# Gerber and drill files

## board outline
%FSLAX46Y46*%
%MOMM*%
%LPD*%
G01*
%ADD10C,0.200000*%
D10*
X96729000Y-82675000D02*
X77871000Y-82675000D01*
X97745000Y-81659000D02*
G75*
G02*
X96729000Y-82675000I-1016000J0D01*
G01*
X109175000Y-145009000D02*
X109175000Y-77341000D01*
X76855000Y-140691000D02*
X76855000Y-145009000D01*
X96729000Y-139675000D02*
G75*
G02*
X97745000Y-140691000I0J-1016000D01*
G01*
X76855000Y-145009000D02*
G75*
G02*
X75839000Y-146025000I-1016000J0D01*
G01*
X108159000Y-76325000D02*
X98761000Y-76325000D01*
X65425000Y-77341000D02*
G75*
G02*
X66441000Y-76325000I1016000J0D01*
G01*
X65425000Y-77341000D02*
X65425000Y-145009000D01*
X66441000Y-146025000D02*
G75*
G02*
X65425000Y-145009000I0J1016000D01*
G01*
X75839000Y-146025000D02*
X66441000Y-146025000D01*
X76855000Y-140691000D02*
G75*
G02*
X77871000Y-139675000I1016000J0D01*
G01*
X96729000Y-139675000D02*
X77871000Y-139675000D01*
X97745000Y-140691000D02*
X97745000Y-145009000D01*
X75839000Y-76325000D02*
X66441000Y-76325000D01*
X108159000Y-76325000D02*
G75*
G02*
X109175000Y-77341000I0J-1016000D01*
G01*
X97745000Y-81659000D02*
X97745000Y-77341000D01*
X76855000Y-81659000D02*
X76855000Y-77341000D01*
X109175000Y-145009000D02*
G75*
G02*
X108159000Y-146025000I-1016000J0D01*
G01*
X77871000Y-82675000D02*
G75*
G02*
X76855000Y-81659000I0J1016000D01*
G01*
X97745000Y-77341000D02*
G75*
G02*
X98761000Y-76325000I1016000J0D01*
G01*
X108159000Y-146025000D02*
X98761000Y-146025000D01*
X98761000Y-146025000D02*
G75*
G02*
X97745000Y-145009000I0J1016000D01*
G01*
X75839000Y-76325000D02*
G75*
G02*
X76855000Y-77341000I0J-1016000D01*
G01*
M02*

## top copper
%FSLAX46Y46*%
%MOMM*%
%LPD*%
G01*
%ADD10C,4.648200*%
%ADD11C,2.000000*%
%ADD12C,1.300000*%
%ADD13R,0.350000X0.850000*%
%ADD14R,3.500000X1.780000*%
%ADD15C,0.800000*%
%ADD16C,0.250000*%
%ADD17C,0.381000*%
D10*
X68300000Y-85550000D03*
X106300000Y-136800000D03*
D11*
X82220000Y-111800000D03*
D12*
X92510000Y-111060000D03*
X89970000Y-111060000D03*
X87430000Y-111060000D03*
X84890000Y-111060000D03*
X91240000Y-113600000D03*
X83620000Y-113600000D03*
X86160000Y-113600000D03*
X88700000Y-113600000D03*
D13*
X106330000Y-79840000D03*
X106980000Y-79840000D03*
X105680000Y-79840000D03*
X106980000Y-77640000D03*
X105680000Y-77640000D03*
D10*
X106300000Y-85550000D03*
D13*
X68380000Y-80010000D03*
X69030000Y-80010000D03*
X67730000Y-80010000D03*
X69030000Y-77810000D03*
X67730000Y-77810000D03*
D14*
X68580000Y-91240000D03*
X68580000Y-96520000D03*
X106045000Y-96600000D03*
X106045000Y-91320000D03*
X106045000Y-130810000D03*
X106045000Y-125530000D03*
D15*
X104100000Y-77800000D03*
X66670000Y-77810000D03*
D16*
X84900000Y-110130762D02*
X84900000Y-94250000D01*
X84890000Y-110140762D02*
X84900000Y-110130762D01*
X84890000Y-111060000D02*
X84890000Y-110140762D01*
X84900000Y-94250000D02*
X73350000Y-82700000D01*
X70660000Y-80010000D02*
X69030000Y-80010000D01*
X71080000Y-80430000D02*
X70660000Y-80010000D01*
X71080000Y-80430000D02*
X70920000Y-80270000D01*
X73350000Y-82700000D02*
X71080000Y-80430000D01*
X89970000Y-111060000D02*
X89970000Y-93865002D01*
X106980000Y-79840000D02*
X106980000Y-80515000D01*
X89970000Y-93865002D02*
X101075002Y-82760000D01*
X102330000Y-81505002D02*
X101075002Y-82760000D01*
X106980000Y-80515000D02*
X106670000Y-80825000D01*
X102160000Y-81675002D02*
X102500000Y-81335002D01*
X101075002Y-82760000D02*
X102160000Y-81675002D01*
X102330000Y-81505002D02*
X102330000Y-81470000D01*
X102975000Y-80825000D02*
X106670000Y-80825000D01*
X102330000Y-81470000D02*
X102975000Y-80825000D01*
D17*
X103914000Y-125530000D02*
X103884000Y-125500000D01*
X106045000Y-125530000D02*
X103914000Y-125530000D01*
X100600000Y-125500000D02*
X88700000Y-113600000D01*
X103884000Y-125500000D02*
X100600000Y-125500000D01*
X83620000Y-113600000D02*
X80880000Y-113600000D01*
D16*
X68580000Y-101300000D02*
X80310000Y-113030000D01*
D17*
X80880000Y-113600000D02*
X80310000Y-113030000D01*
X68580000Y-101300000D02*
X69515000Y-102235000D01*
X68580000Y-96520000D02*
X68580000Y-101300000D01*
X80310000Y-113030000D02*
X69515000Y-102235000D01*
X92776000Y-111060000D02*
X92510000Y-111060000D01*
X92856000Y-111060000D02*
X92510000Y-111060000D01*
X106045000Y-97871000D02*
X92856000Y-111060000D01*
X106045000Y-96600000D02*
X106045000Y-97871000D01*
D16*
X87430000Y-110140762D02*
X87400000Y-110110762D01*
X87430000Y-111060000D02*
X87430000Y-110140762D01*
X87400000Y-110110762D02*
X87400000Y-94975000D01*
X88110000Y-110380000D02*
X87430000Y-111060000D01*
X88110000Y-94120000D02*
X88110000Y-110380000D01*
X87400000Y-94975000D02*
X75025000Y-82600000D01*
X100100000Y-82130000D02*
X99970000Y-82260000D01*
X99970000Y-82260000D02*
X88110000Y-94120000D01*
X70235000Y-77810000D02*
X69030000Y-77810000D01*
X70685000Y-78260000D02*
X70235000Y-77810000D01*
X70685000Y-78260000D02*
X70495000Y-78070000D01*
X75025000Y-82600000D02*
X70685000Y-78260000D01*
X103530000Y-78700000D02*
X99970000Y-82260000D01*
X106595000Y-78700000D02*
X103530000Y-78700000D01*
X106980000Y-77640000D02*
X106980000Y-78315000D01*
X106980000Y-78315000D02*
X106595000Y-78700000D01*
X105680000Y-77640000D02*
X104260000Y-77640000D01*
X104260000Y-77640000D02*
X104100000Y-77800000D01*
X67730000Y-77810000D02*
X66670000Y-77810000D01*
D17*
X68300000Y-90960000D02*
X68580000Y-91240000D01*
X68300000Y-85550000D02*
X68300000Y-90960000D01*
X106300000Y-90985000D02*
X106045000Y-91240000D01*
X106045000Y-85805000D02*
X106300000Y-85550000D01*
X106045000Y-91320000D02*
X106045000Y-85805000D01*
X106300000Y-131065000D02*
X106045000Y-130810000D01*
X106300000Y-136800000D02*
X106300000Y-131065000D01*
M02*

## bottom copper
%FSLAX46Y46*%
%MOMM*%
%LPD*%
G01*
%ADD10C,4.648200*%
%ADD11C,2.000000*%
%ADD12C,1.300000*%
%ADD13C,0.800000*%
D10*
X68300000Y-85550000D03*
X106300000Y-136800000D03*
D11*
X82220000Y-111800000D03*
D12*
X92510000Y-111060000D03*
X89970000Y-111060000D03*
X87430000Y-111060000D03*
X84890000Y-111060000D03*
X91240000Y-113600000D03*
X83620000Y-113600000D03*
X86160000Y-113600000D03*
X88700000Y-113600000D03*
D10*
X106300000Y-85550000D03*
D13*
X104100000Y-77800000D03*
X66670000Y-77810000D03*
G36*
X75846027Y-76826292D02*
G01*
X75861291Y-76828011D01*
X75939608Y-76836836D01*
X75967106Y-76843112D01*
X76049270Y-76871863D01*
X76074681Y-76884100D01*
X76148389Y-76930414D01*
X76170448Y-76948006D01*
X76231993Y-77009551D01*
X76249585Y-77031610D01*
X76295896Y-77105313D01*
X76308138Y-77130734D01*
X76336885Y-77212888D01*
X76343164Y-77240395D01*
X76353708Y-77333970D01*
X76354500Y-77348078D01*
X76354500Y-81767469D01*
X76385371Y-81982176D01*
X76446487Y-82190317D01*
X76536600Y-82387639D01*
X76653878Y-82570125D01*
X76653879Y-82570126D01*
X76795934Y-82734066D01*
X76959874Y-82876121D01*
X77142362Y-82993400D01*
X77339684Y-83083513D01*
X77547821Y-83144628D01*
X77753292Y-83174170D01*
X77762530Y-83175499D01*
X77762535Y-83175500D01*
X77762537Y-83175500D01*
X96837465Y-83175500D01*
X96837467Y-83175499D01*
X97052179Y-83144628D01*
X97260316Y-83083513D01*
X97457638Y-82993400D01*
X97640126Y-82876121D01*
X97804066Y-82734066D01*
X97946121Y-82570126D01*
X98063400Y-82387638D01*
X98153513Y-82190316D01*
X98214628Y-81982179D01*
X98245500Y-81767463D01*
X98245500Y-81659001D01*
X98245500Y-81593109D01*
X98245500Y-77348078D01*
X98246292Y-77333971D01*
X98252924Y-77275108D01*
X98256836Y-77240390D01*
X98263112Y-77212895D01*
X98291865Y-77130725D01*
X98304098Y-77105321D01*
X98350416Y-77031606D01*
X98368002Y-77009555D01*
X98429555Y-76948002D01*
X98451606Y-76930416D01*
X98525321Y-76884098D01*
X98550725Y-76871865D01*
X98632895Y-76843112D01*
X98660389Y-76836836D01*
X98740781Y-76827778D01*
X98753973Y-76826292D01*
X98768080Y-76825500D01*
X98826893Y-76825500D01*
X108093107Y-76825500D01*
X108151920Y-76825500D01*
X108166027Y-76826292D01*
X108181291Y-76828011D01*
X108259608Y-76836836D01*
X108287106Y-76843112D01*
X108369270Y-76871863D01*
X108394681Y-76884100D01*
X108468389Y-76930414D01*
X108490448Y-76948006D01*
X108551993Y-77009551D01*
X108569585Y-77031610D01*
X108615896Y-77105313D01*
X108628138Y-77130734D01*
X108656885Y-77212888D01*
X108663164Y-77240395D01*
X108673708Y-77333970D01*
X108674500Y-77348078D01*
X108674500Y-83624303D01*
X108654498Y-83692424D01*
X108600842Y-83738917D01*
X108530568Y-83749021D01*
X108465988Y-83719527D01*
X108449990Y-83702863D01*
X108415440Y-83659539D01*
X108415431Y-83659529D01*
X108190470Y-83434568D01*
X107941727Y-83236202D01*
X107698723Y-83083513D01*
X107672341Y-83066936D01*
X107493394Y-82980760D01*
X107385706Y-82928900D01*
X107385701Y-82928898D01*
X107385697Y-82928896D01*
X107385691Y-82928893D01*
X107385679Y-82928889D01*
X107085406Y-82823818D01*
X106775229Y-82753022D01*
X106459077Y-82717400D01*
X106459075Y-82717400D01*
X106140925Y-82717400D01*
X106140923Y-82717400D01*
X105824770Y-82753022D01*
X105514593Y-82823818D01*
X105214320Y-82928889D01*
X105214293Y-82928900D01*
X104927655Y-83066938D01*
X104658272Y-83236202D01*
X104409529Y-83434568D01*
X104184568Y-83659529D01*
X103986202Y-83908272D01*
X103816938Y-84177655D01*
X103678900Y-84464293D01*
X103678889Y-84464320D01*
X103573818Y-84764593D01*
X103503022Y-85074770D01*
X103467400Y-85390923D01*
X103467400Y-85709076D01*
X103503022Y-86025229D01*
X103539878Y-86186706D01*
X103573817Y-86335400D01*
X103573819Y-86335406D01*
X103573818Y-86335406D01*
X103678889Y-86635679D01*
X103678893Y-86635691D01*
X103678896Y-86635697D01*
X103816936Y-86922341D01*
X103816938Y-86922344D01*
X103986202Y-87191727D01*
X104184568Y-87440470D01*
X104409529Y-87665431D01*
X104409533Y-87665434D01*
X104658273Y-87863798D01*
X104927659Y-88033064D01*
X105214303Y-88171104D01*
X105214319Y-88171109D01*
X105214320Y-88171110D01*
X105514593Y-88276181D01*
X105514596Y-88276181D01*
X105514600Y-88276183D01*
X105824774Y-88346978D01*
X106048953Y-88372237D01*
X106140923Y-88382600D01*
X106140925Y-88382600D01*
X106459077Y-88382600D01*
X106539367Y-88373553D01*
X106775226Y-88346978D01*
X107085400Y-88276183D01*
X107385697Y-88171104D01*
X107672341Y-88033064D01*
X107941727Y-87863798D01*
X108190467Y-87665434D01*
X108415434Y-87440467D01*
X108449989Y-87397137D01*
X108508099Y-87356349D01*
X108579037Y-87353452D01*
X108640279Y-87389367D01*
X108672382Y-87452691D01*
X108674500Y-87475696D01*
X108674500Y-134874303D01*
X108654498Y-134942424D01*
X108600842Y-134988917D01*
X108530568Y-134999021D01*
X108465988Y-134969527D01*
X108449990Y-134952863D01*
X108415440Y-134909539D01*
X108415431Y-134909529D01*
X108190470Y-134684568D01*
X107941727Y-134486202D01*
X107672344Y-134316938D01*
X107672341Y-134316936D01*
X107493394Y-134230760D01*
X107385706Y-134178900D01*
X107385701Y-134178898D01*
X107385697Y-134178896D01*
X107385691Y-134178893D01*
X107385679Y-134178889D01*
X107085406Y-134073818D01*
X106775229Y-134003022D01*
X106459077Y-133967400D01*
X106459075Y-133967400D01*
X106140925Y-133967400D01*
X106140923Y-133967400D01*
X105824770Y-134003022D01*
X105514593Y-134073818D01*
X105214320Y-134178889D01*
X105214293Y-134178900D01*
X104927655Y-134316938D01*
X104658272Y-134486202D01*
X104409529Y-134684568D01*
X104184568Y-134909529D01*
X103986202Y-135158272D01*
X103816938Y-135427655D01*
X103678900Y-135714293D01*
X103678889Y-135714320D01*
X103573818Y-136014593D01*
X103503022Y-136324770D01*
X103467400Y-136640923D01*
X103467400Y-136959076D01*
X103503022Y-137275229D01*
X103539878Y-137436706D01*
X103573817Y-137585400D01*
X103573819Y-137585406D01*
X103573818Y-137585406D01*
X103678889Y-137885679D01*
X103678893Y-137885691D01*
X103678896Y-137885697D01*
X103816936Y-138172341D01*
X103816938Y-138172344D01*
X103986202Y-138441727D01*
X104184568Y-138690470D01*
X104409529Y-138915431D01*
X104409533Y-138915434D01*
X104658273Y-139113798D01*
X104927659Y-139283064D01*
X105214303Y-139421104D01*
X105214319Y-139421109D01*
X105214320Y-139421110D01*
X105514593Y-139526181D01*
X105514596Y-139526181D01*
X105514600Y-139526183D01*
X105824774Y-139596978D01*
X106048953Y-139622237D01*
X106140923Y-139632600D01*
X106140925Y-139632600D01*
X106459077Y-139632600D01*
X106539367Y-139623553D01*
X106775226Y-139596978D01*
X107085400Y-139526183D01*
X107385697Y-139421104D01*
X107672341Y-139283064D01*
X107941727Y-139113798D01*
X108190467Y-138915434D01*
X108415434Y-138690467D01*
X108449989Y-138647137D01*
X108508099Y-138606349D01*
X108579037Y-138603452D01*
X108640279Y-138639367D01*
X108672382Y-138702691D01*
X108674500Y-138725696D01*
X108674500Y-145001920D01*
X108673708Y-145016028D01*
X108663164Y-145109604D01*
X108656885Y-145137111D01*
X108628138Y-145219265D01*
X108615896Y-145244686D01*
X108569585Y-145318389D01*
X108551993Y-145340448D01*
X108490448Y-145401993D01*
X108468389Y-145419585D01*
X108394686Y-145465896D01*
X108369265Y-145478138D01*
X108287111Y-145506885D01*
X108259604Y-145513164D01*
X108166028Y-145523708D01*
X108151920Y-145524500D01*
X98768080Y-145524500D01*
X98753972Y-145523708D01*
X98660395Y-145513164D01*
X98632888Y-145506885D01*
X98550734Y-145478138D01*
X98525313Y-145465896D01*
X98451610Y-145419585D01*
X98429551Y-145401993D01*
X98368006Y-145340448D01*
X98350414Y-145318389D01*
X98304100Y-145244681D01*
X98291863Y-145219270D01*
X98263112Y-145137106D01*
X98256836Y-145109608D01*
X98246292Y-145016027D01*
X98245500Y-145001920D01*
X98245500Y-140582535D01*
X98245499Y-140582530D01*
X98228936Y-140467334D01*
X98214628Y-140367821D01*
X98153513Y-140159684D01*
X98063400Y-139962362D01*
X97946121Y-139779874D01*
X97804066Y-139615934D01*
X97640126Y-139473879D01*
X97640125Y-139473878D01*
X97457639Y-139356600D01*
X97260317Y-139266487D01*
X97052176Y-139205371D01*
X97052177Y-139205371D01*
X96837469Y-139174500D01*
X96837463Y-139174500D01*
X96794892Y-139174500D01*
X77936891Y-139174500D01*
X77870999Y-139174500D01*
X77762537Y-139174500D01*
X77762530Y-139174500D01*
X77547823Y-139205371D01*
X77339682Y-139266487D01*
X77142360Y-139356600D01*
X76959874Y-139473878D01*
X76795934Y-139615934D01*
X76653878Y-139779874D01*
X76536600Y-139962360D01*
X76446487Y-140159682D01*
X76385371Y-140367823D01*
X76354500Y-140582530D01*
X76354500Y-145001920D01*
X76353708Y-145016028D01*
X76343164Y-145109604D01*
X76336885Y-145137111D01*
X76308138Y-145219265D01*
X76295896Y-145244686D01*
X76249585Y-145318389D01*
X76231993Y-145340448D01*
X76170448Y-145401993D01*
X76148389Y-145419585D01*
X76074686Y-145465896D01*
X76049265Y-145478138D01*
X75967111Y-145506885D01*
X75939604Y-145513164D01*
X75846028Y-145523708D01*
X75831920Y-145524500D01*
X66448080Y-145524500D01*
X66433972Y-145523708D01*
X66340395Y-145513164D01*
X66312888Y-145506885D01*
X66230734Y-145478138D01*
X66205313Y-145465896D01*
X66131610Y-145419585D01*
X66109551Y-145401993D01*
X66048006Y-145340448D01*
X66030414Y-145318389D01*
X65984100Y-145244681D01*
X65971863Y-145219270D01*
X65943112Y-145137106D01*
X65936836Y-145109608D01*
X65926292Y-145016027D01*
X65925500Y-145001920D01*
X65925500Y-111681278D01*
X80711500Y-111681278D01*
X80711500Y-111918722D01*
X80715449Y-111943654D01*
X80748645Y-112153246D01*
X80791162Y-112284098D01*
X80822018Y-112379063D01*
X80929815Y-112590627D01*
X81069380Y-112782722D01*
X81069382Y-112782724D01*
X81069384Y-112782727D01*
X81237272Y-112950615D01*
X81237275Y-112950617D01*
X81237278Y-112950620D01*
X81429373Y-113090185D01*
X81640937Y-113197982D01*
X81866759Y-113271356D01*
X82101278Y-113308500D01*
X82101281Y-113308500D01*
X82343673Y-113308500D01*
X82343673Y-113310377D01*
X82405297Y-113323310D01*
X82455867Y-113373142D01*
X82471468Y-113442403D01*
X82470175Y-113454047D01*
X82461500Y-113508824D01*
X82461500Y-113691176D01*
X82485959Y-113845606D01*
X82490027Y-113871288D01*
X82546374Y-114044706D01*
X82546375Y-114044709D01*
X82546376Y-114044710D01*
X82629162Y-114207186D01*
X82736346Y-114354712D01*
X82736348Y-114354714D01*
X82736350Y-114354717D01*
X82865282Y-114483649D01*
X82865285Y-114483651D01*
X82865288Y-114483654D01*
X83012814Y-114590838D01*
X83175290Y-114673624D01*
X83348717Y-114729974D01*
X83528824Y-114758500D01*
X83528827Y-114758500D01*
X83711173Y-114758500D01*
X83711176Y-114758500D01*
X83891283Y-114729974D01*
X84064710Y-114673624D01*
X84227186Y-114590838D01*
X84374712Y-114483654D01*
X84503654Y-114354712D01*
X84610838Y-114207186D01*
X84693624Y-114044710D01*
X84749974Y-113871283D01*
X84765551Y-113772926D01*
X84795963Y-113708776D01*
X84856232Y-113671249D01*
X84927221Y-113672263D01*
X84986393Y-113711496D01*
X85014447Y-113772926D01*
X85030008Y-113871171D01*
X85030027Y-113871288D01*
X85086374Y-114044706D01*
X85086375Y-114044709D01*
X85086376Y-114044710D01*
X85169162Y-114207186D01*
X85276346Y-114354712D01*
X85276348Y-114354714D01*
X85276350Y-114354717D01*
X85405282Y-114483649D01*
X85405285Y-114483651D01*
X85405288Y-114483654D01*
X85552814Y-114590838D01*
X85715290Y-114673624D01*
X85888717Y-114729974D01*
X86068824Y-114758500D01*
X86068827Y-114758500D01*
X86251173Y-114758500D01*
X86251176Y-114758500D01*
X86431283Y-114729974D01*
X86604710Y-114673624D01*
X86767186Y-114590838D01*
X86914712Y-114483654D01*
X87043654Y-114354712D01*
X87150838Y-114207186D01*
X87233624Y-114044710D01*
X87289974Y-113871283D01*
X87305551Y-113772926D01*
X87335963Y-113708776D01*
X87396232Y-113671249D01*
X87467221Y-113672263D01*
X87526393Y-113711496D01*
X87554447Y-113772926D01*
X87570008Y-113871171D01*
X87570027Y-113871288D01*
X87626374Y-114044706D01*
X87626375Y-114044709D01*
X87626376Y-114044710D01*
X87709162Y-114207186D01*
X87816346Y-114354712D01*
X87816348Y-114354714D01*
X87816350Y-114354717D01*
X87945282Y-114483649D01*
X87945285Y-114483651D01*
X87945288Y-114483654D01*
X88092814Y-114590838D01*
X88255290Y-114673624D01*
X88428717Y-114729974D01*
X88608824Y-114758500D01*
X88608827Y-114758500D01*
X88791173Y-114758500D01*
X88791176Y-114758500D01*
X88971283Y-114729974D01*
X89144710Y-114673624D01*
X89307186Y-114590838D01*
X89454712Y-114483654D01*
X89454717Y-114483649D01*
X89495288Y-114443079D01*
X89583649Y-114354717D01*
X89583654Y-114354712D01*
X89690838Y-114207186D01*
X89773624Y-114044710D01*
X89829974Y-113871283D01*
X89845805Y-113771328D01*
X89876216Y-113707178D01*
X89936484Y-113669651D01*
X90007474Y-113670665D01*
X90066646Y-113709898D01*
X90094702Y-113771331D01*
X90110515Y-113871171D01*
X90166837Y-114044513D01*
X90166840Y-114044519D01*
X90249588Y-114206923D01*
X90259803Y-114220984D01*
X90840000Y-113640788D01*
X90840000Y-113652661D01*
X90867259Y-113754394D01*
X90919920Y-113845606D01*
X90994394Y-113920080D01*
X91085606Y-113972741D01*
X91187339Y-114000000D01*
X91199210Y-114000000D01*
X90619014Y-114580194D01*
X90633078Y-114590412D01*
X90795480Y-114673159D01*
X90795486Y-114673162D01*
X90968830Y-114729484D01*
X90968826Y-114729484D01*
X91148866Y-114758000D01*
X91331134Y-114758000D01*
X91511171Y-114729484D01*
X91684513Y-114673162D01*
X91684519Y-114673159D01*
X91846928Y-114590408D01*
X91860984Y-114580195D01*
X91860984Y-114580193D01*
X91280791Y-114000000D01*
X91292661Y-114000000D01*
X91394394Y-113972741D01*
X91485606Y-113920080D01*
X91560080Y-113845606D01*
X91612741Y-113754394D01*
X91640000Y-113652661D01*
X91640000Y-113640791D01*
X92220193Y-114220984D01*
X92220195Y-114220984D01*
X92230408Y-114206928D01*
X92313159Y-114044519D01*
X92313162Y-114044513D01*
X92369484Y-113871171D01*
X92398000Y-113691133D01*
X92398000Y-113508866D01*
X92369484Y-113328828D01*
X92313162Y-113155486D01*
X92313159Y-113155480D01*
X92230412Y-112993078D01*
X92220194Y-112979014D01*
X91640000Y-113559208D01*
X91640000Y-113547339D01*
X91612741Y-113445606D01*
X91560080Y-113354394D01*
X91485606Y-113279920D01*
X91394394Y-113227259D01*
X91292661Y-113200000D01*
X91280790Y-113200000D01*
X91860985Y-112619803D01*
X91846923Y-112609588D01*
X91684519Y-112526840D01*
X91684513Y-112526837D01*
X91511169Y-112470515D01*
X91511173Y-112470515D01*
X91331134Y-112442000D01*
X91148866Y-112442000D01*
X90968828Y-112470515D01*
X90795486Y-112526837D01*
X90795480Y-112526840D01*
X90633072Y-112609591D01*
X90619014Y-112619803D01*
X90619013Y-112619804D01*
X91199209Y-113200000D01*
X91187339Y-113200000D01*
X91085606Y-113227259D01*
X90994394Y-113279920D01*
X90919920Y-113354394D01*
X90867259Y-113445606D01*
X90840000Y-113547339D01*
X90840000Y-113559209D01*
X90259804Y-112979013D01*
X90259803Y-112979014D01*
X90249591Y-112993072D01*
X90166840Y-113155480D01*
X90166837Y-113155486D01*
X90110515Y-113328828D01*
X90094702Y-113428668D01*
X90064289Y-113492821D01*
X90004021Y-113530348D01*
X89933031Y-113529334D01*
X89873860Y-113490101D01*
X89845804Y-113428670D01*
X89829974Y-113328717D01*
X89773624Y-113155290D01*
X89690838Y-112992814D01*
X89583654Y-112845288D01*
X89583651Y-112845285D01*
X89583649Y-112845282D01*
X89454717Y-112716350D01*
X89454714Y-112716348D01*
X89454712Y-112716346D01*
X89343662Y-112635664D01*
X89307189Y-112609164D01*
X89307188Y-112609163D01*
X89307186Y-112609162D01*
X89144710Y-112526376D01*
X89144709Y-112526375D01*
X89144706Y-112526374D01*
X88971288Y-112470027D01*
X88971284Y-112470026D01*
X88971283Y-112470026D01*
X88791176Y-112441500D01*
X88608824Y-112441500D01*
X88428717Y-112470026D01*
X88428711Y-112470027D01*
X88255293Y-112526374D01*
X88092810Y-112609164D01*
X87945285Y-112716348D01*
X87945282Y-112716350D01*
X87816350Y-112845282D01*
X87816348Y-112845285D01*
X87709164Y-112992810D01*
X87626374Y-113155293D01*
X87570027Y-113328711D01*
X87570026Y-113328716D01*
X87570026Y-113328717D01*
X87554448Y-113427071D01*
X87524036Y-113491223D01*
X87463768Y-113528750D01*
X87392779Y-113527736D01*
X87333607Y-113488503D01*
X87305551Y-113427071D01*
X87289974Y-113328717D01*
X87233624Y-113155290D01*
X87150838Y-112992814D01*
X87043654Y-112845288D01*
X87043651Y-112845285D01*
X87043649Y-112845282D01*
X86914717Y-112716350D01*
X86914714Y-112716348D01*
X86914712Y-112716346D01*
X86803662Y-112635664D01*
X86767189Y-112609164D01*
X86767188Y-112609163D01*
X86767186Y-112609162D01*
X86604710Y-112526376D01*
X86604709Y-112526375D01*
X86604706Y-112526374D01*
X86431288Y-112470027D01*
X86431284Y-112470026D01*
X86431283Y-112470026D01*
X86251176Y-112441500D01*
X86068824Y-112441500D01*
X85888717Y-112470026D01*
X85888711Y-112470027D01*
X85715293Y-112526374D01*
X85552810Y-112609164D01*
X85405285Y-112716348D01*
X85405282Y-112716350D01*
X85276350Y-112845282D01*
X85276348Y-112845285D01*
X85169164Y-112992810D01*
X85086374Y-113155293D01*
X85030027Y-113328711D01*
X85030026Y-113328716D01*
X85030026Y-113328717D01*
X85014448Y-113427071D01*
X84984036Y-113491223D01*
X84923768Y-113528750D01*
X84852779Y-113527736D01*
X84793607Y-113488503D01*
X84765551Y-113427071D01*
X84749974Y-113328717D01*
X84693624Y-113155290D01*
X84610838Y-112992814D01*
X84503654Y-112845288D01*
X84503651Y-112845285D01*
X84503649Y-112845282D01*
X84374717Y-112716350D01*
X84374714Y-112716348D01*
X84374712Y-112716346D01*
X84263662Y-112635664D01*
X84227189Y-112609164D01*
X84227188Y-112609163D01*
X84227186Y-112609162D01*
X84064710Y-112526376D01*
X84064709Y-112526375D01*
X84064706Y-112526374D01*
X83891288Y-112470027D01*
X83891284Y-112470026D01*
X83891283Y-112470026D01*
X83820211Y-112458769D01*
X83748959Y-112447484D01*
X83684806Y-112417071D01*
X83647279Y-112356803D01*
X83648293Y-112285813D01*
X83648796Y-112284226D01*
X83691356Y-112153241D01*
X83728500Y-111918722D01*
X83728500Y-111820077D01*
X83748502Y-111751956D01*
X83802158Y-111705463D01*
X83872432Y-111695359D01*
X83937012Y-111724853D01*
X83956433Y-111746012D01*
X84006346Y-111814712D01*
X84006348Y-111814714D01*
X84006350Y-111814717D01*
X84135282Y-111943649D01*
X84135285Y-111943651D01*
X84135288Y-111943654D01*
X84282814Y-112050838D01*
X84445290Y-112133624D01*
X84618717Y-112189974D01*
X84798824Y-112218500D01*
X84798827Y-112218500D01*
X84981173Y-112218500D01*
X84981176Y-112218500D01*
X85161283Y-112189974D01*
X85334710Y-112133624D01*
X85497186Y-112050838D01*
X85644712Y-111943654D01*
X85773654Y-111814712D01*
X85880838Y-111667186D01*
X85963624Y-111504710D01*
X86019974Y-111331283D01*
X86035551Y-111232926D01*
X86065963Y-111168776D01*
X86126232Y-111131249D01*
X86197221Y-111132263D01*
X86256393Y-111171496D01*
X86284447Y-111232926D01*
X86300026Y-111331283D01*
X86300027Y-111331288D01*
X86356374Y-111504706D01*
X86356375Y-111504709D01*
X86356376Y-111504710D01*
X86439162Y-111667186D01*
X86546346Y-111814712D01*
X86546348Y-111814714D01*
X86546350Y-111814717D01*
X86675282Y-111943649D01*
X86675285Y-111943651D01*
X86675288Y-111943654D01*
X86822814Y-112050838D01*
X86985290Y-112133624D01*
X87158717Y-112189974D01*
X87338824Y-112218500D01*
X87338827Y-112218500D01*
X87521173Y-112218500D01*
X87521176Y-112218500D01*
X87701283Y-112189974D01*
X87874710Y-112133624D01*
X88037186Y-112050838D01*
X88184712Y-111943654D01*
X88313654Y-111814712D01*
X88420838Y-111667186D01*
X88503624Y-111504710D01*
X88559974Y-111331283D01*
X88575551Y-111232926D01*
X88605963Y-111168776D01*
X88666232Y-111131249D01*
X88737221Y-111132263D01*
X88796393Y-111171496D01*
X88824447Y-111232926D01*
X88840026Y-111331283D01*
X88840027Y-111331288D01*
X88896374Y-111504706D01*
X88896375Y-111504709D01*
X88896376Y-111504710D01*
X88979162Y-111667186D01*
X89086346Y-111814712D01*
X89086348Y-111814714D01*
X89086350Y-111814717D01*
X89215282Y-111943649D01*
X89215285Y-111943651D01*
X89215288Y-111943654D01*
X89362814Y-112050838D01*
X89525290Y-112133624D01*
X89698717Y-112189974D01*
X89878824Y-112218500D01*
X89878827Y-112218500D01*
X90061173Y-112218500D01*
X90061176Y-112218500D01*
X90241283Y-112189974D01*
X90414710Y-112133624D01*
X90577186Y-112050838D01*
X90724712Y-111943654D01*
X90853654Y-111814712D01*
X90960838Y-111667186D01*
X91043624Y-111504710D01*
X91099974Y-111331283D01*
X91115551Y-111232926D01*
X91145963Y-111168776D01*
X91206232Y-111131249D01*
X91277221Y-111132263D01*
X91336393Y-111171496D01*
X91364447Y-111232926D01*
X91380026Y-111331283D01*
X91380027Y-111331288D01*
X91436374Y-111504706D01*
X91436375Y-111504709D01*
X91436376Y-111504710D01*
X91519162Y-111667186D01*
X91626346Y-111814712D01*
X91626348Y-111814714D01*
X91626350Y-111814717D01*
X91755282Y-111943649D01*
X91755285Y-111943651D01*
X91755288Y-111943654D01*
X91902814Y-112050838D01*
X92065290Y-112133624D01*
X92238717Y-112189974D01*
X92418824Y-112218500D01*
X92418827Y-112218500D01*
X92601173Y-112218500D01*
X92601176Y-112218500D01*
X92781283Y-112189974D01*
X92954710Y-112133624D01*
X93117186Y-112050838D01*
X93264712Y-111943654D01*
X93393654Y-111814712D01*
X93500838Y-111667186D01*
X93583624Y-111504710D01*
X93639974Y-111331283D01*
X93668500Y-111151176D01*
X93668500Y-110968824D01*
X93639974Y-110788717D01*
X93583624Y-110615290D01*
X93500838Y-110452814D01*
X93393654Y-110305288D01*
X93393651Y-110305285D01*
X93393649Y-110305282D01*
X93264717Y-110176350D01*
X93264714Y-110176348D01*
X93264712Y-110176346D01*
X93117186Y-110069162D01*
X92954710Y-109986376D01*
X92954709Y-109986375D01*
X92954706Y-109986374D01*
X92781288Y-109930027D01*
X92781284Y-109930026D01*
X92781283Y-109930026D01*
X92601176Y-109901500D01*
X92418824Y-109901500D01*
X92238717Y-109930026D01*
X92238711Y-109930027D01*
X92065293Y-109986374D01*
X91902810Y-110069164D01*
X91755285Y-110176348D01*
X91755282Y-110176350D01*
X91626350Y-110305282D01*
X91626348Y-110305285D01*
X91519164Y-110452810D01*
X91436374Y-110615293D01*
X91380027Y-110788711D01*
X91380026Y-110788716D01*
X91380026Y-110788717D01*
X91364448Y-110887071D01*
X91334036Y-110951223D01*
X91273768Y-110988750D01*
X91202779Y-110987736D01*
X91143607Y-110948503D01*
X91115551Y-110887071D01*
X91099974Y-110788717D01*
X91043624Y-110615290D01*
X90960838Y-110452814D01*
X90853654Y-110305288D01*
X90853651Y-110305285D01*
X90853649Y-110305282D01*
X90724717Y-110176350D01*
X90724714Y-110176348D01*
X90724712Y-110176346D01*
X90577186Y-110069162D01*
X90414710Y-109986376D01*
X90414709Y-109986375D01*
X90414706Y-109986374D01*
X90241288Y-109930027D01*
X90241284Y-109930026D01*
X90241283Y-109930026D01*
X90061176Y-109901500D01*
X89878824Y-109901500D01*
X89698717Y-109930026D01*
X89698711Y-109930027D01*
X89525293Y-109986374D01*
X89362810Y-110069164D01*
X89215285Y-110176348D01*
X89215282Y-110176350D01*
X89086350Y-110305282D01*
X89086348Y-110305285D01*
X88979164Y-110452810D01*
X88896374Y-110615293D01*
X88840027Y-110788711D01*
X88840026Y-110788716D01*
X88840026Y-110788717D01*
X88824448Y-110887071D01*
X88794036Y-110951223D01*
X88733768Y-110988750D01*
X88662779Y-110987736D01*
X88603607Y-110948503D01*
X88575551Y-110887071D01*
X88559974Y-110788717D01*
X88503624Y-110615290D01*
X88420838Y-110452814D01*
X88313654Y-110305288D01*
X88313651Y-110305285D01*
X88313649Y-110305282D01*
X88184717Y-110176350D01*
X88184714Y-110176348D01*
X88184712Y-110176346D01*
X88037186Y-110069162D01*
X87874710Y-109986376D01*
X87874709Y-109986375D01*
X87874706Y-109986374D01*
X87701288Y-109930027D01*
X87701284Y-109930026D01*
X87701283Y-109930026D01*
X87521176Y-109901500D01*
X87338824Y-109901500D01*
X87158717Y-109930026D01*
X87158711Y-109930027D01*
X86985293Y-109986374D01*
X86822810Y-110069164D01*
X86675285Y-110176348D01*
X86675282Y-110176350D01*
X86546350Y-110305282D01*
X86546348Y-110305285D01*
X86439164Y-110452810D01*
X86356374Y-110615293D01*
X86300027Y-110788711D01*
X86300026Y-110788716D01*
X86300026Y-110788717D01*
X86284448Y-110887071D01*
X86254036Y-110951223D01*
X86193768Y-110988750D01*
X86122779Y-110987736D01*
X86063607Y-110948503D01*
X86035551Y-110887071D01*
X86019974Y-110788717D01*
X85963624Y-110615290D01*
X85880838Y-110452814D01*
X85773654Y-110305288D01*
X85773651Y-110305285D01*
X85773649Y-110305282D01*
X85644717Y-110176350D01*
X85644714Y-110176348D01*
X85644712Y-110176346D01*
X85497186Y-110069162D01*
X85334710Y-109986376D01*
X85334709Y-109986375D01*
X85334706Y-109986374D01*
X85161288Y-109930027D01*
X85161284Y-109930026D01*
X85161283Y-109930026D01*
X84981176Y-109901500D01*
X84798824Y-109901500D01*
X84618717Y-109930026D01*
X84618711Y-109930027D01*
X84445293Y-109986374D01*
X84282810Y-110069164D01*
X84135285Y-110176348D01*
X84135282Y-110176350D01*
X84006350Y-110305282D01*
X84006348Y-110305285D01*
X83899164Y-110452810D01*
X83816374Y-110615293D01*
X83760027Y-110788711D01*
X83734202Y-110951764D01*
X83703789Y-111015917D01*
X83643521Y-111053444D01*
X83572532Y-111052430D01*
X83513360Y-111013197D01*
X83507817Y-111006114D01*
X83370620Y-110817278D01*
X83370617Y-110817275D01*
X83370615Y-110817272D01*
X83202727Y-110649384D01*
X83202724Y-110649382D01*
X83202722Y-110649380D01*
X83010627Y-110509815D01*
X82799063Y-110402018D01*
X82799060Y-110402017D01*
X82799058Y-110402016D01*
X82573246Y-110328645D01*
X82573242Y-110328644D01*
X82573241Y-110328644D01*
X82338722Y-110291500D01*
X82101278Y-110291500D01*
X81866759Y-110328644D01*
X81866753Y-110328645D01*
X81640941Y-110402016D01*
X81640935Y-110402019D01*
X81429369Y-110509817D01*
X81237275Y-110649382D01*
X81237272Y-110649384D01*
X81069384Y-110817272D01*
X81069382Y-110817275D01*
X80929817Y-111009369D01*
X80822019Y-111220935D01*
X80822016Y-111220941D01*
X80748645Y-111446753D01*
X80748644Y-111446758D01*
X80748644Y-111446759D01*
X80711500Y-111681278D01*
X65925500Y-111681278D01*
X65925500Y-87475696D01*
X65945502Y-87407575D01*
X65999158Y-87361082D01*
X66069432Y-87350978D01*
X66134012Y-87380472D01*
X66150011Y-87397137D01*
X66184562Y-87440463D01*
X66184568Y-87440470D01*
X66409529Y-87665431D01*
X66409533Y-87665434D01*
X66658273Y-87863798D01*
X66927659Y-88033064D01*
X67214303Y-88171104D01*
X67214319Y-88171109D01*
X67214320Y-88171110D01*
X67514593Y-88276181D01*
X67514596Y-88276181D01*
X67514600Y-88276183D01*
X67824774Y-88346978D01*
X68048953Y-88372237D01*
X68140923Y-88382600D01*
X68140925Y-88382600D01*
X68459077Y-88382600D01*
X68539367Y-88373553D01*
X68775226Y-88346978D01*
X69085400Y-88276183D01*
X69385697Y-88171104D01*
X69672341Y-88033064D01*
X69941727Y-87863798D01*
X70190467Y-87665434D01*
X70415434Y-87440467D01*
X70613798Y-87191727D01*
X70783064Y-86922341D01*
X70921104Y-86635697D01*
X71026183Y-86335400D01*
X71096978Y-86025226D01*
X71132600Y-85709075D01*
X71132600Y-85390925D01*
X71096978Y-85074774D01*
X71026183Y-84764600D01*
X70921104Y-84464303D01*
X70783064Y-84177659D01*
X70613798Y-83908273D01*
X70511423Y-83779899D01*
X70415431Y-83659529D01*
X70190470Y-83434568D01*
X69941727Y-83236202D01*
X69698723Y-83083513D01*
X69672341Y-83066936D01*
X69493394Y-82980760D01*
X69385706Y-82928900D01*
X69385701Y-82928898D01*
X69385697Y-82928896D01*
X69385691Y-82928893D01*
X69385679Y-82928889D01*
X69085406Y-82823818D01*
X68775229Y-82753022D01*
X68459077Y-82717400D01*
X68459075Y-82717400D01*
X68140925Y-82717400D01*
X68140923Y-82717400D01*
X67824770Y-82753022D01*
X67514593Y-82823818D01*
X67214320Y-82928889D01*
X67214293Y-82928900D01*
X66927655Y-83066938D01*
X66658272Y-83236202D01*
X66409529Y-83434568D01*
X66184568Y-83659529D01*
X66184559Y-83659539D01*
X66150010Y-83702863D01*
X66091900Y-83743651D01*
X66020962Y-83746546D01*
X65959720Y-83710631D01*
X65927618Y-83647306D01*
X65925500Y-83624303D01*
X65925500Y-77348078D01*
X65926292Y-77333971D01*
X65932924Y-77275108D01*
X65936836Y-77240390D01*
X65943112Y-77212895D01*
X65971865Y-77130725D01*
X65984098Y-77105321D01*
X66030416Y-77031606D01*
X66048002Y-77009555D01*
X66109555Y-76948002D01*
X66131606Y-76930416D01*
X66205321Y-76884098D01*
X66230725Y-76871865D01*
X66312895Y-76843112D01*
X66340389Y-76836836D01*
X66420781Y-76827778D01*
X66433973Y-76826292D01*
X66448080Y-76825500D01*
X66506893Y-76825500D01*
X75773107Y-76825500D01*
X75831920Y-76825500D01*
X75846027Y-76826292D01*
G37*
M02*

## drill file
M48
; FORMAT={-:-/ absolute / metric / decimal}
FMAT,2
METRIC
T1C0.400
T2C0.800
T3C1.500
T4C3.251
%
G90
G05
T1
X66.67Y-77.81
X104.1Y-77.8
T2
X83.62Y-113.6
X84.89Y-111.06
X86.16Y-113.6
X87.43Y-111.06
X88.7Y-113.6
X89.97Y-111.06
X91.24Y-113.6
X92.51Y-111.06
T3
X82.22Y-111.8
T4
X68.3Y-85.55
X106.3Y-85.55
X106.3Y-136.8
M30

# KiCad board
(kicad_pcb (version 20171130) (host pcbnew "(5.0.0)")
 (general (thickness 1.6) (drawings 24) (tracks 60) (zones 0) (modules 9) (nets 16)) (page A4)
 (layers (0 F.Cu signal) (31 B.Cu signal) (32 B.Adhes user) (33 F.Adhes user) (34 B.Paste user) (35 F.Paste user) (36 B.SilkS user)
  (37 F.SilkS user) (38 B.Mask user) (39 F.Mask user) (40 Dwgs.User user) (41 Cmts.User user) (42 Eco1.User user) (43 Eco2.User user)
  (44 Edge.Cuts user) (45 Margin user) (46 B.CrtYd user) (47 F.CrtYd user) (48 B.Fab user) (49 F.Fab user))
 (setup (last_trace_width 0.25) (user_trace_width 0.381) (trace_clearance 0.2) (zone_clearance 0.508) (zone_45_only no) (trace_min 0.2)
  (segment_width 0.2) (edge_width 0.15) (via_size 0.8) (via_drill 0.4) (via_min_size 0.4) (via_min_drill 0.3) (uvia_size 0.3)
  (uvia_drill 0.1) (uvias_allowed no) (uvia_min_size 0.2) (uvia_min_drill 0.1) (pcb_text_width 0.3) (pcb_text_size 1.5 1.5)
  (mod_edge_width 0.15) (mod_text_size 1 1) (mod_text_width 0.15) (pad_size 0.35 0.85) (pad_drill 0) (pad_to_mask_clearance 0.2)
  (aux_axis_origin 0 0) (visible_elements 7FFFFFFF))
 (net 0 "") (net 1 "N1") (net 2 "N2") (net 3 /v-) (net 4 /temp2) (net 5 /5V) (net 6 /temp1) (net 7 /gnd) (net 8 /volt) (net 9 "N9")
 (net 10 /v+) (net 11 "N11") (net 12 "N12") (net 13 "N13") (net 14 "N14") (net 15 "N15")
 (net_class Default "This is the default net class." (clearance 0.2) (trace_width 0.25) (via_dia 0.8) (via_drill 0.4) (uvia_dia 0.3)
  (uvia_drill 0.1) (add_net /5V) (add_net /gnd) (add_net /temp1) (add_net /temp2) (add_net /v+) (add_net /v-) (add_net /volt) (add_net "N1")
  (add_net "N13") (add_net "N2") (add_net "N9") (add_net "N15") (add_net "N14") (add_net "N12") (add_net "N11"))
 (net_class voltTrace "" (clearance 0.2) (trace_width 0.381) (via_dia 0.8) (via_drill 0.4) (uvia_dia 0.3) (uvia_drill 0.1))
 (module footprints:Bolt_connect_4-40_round (layer F.Cu) (at 68.3 85.55)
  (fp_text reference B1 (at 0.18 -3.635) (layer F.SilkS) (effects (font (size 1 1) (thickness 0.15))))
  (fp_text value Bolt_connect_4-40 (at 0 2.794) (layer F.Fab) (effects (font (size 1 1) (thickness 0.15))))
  (pad 1 thru_hole circle (at 0 0) (size 4.6482 4.6482) (drill 3.2512) (layers *.Cu *.Mask) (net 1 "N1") (clearance 0.508)))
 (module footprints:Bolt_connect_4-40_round (layer F.Cu) (at 106.3 136.8)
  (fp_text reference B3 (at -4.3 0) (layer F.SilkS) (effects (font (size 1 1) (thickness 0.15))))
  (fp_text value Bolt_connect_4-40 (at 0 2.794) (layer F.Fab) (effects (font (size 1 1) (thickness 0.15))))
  (pad 1 thru_hole circle (at 0 0) (size 4.6482 4.6482) (drill 3.2512) (layers *.Cu *.Mask) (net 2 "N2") (clearance 0.508)))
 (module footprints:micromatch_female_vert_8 (layer F.Cu) (at 88.7 113.6 90)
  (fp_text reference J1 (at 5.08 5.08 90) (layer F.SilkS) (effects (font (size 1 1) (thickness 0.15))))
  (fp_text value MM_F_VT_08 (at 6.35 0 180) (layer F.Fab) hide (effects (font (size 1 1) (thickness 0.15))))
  (pad 9 thru_hole circle (at 1.8 -6.48 90) (size 2 2) (drill 1.5) (layers *.Cu *.Mask))
  (pad 8 thru_hole circle (at 2.54 3.81 90) (size 1.3 1.3) (drill 0.8) (layers *.Cu *.Mask) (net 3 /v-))
  (pad 6 thru_hole circle (at 2.54 1.27 90) (size 1.3 1.3) (drill 0.8) (layers *.Cu *.Mask) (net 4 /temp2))
  (pad 4 thru_hole circle (at 2.54 -1.27 90) (size 1.3 1.3) (drill 0.8) (layers *.Cu *.Mask) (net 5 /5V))
  (pad 2 thru_hole circle (at 2.54 -3.81 90) (size 1.3 1.3) (drill 0.8) (layers *.Cu *.Mask) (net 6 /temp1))
  (pad 7 thru_hole circle (at 0 2.54 90) (size 1.3 1.3) (drill 0.8) (layers *.Cu *.Mask) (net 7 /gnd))
  (pad 1 thru_hole circle (at 0 -5.08 90) (size 1.3 1.3) (drill 0.8) (layers *.Cu *.Mask) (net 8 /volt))
  (pad 3 thru_hole circle (at 0 -2.54 90) (size 1.3 1.3) (drill 0.8) (layers *.Cu *.Mask) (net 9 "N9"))
  (pad 5 thru_hole circle (at 0 0 90) (size 1.3 1.3) (drill 0.8) (layers *.Cu *.Mask) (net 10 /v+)))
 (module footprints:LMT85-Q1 (layer F.Cu) (at 105.68 79.84)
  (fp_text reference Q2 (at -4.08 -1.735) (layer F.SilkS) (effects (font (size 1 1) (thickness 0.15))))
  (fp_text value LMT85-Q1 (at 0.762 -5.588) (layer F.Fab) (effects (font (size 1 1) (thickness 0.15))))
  (pad 3 smd rect (at 0.65 0) (size 0.35 0.85) (layers F.Cu F.Paste F.Mask) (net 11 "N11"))
  (pad 4 smd rect (at 1.3 0) (size 0.35 0.85) (layers F.Cu F.Paste F.Mask) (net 4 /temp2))
  (pad 2 smd rect (at 0 0) (size 0.35 0.85) (layers F.Cu F.Paste F.Mask) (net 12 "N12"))
  (pad 5 smd rect (at 1.3 -2.2) (size 0.35 0.85) (layers F.Cu F.Paste F.Mask) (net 5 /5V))
  (pad 1 smd rect (at 0 -2.2) (size 0.35 0.85) (layers F.Cu F.Paste F.Mask) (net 7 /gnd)))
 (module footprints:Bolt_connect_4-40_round (layer F.Cu) (at 106.3 85.55)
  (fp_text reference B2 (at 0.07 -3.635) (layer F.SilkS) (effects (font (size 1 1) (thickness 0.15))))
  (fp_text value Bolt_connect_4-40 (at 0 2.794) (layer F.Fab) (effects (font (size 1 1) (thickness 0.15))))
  (pad 1 thru_hole circle (at 0 0) (size 4.6482 4.6482) (drill 3.2512) (layers *.Cu *.Mask) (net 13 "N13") (clearance 0.508)))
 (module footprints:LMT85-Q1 (layer F.Cu) (at 67.73 80.01)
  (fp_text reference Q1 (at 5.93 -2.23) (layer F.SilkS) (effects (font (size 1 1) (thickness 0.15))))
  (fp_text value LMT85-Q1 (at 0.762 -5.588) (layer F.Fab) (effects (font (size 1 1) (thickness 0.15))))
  (pad 3 smd rect (at 0.65 0) (size 0.35 0.85) (layers F.Cu F.Paste F.Mask) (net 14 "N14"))
  (pad 4 smd rect (at 1.3 0) (size 0.35 0.85) (layers F.Cu F.Paste F.Mask) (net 6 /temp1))
  (pad 2 smd rect (at 0 0) (size 0.35 0.85) (layers F.Cu F.Paste F.Mask) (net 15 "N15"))
  (pad 5 smd rect (at 1.3 -2.2) (size 0.35 0.85) (layers F.Cu F.Paste F.Mask) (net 5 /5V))
  (pad 1 smd rect (at 0 -2.2) (size 0.35 0.85) (layers F.Cu F.Paste F.Mask) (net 7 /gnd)))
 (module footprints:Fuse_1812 (layer F.Cu) (at 68.58 96.52 90)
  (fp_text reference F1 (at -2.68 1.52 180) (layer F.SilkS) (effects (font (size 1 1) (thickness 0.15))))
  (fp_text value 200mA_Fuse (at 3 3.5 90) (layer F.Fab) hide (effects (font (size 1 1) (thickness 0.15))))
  (pad 2 smd rect (at 5.28 0 90) (size 1.78 3.5) (layers F.Cu F.Paste F.Mask) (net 1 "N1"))
  (pad 1 smd rect (at 0 0 90) (size 1.78 3.5) (layers F.Cu F.Paste F.Mask) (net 8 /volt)))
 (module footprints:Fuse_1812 (layer F.Cu) (at 106.045 96.6 90)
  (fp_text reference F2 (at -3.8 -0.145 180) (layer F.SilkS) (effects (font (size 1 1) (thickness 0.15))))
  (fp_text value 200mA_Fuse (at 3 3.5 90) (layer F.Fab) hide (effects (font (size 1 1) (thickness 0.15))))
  (pad 1 smd rect (at 0 0 90) (size 1.78 3.5) (layers F.Cu F.Paste F.Mask) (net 3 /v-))
  (pad 2 smd rect (at 5.28 0 90) (size 1.78 3.5) (layers F.Cu F.Paste F.Mask) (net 13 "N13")))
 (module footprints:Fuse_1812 (layer F.Cu) (at 106.045 125.53 270)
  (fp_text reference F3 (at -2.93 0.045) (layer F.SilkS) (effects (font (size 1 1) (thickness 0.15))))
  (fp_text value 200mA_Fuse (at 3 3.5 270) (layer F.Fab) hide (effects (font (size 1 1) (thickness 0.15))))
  (pad 2 smd rect (at 5.28 0 270) (size 1.78 3.5) (layers F.Cu F.Paste F.Mask) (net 2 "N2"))
  (pad 1 smd rect (at 0 0 270) (size 1.78 3.5) (layers F.Cu F.Paste F.Mask) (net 10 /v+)))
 (gr_line (start 96.729 82.675) (end 77.871 82.675) (layer Edge.Cuts) (width 0.2))
 (gr_arc (start 96.729 81.659) (end 96.729 82.675) (angle -90) (layer Edge.Cuts) (width 0.2))
 (gr_line (start 109.175 145.009) (end 109.175 77.341) (layer Edge.Cuts) (width 0.2))
 (gr_line (start 76.855 140.691) (end 76.855 145.009) (layer Edge.Cuts) (width 0.2))
 (gr_arc (start 96.729 140.691) (end 97.745 140.691) (angle -90) (layer Edge.Cuts) (width 0.2))
 (gr_arc (start 75.839 145.009) (end 75.839 146.025) (angle -90) (layer Edge.Cuts) (width 0.2))
 (gr_line (start 108.159 76.325) (end 98.761 76.325) (layer Edge.Cuts) (width 0.2))
 (gr_arc (start 66.441 77.341) (end 66.441 76.325) (angle -90) (layer Edge.Cuts) (width 0.2))
 (gr_line (start 65.425 77.341) (end 65.425 145.009) (layer Edge.Cuts) (width 0.2))
 (gr_arc (start 66.441 145.009) (end 65.425 145.009) (angle -90) (layer Edge.Cuts) (width 0.2))
 (gr_line (start 75.839 146.025) (end 66.441 146.025) (layer Edge.Cuts) (width 0.2))
 (gr_arc (start 77.871 140.691) (end 77.871 139.675) (angle -90) (layer Edge.Cuts) (width 0.2))
 (gr_line (start 96.729 139.675) (end 77.871 139.675) (layer Edge.Cuts) (width 0.2))
 (gr_line (start 97.745 140.691) (end 97.745 145.009) (layer Edge.Cuts) (width 0.2))
 (gr_line (start 75.839 76.325) (end 66.441 76.325) (layer Edge.Cuts) (width 0.2))
 (gr_arc (start 108.159 77.341) (end 109.175 77.341) (angle -90) (layer Edge.Cuts) (width 0.2))
 (gr_line (start 97.745 81.659) (end 97.745 77.341) (layer Edge.Cuts) (width 0.2))
 (gr_line (start 76.855 81.659) (end 76.855 77.341) (layer Edge.Cuts) (width 0.2))
 (gr_arc (start 108.159 145.009) (end 108.159 146.025) (angle -90) (layer Edge.Cuts) (width 0.2))
 (gr_arc (start 77.871 81.659) (end 76.855 81.659) (angle -90) (layer Edge.Cuts) (width 0.2))
 (gr_arc (start 98.761 77.341) (end 98.761 76.325) (angle -90) (layer Edge.Cuts) (width 0.2))
 (gr_line (start 108.159 146.025) (end 98.761 146.025) (layer Edge.Cuts) (width 0.2))
 (gr_arc (start 98.761 145.009) (end 97.745 145.009) (angle -90) (layer Edge.Cuts) (width 0.2))
 (gr_arc (start 75.839 77.341) (end 76.855 77.341) (angle -90) (layer Edge.Cuts) (width 0.2))
 (segment (start 84.9 110.130762) (end 84.9 94.25) (width 0.25) (layer F.Cu) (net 6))
 (segment (start 84.89 110.140762) (end 84.9 110.130762) (width 0.25) (layer F.Cu) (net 6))
 (segment (start 84.89 111.06) (end 84.89 110.140762) (width 0.25) (layer F.Cu) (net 6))
 (segment (start 84.9 94.25) (end 73.35 82.7) (width 0.25) (layer F.Cu) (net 6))
 (segment (start 70.66 80.01) (end 69.03 80.01) (width 0.25) (layer F.Cu) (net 6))
 (segment (start 71.08 80.43) (end 70.66 80.01) (width 0.25) (layer F.Cu) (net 6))
 (segment (start 71.08 80.43) (end 70.92 80.27) (width 0.25) (layer F.Cu) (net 6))
 (segment (start 73.35 82.7) (end 71.08 80.43) (width 0.25) (layer F.Cu) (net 6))
 (segment (start 89.97 111.06) (end 89.97 93.865002) (width 0.25) (layer F.Cu) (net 4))
 (segment (start 106.98 79.84) (end 106.98 80.515) (width 0.25) (layer F.Cu) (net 4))
 (segment (start 89.97 93.865002) (end 101.075002 82.76) (width 0.25) (layer F.Cu) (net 4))
 (segment (start 102.33 81.505002) (end 101.075002 82.76) (width 0.25) (layer F.Cu) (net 4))
 (segment (start 106.98 80.515) (end 106.67 80.825) (width 0.25) (layer F.Cu) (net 4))
 (segment (start 102.16 81.675002) (end 102.5 81.335002) (width 0.25) (layer F.Cu) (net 4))
 (segment (start 101.075002 82.76) (end 102.16 81.675002) (width 0.25) (layer F.Cu) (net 4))
 (segment (start 102.33 81.505002) (end 102.33 81.47) (width 0.25) (layer F.Cu) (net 4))
 (segment (start 102.975 80.825) (end 106.67 80.825) (width 0.25) (layer F.Cu) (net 4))
 (segment (start 102.33 81.47) (end 102.975 80.825) (width 0.25) (layer F.Cu) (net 4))
 (segment (start 103.914 125.53) (end 103.884 125.5) (width 0.381) (layer F.Cu) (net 10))
 (segment (start 106.045 125.53) (end 103.914 125.53) (width 0.381) (layer F.Cu) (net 10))
 (segment (start 100.6 125.5) (end 88.7 113.6) (width 0.381) (layer F.Cu) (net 10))
 (segment (start 103.884 125.5) (end 100.6 125.5) (width 0.381) (layer F.Cu) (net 10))
 (segment (start 83.62 113.6) (end 80.88 113.6) (width 0.381) (layer F.Cu) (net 8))
 (segment (start 68.58 101.3) (end 80.31 113.03) (width 0.25) (layer F.Cu) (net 8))
 (segment (start 80.88 113.6) (end 80.31 113.03) (width 0.381) (layer F.Cu) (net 8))
 (segment (start 68.58 101.3) (end 69.515 102.235) (width 0.381) (layer F.Cu) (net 8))
 (segment (start 68.58 96.52) (end 68.58 101.3) (width 0.381) (layer F.Cu) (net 8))
 (segment (start 80.31 113.03) (end 69.515 102.235) (width 0.381) (layer F.Cu) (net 8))
 (segment (start 92.776 111.06) (end 92.51 111.06) (width 0.381) (layer F.Cu) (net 3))
 (segment (start 92.856 111.06) (end 92.51 111.06) (width 0.381) (layer F.Cu) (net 3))
 (segment (start 106.045 97.871) (end 92.856 111.06) (width 0.381) (layer F.Cu) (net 3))
 (segment (start 106.045 96.6) (end 106.045 97.871) (width 0.381) (layer F.Cu) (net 3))
 (segment (start 87.43 110.140762) (end 87.4 110.110762) (width 0.25) (layer F.Cu) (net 5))
 (segment (start 87.43 111.06) (end 87.43 110.140762) (width 0.25) (layer F.Cu) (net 5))
 (segment (start 87.4 110.110762) (end 87.4 94.975) (width 0.25) (layer F.Cu) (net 5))
 (segment (start 88.11 110.38) (end 87.43 111.06) (width 0.25) (layer F.Cu) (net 5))
 (segment (start 88.11 94.12) (end 88.11 110.38) (width 0.25) (layer F.Cu) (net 5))
 (segment (start 87.4 94.975) (end 75.025 82.6) (width 0.25) (layer F.Cu) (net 5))
 (segment (start 100.1 82.13) (end 99.97 82.26) (width 0.25) (layer F.Cu) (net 5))
 (segment (start 99.97 82.26) (end 88.11 94.12) (width 0.25) (layer F.Cu) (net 5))
 (segment (start 70.235 77.81) (end 69.03 77.81) (width 0.25) (layer F.Cu) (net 5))
 (segment (start 70.685 78.26) (end 70.235 77.81) (width 0.25) (layer F.Cu) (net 5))
 (segment (start 70.685 78.26) (end 70.495 78.07) (width 0.25) (layer F.Cu) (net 5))
 (segment (start 75.025 82.6) (end 70.685 78.26) (width 0.25) (layer F.Cu) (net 5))
 (segment (start 103.53 78.7) (end 99.97 82.26) (width 0.25) (layer F.Cu) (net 5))
 (segment (start 106.595 78.7) (end 103.53 78.7) (width 0.25) (layer F.Cu) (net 5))
 (segment (start 106.98 77.64) (end 106.98 78.315) (width 0.25) (layer F.Cu) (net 5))
 (segment (start 106.98 78.315) (end 106.595 78.7) (width 0.25) (layer F.Cu) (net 5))
 (via (at 104.1 77.8) (size 0.8) (drill 0.4) (layers F.Cu B.Cu) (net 7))
 (segment (start 105.68 77.64) (end 104.26 77.64) (width 0.25) (layer F.Cu) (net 7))
 (segment (start 104.26 77.64) (end 104.1 77.8) (width 0.25) (layer F.Cu) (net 7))
 (via (at 66.67 77.81) (size 0.8) (drill 0.4) (layers F.Cu B.Cu) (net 7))
 (segment (start 67.73 77.81) (end 66.67 77.81) (width 0.25) (layer F.Cu) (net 7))
 (segment (start 68.3 90.96) (end 68.58 91.24) (width 0.381) (layer F.Cu) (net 1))
 (segment (start 68.3 85.55) (end 68.3 90.96) (width 0.381) (layer F.Cu) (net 1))
 (segment (start 106.3 90.985) (end 106.045 91.24) (width 0.381) (layer F.Cu) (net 13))
 (segment (start 106.045 85.805) (end 106.3 85.55) (width 0.381) (layer F.Cu) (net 13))
 (segment (start 106.045 91.32) (end 106.045 85.805) (width 0.381) (layer F.Cu) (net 13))
 (segment (start 106.3 131.065) (end 106.045 130.81) (width 0.381) (layer F.Cu) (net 2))
 (segment (start 106.3 136.8) (end 106.3 131.065) (width 0.381) (layer F.Cu) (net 2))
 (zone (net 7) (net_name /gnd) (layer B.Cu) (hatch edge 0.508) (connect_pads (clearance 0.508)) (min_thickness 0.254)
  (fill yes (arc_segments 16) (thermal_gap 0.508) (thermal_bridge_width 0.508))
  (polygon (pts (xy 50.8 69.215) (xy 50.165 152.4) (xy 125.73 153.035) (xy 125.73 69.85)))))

